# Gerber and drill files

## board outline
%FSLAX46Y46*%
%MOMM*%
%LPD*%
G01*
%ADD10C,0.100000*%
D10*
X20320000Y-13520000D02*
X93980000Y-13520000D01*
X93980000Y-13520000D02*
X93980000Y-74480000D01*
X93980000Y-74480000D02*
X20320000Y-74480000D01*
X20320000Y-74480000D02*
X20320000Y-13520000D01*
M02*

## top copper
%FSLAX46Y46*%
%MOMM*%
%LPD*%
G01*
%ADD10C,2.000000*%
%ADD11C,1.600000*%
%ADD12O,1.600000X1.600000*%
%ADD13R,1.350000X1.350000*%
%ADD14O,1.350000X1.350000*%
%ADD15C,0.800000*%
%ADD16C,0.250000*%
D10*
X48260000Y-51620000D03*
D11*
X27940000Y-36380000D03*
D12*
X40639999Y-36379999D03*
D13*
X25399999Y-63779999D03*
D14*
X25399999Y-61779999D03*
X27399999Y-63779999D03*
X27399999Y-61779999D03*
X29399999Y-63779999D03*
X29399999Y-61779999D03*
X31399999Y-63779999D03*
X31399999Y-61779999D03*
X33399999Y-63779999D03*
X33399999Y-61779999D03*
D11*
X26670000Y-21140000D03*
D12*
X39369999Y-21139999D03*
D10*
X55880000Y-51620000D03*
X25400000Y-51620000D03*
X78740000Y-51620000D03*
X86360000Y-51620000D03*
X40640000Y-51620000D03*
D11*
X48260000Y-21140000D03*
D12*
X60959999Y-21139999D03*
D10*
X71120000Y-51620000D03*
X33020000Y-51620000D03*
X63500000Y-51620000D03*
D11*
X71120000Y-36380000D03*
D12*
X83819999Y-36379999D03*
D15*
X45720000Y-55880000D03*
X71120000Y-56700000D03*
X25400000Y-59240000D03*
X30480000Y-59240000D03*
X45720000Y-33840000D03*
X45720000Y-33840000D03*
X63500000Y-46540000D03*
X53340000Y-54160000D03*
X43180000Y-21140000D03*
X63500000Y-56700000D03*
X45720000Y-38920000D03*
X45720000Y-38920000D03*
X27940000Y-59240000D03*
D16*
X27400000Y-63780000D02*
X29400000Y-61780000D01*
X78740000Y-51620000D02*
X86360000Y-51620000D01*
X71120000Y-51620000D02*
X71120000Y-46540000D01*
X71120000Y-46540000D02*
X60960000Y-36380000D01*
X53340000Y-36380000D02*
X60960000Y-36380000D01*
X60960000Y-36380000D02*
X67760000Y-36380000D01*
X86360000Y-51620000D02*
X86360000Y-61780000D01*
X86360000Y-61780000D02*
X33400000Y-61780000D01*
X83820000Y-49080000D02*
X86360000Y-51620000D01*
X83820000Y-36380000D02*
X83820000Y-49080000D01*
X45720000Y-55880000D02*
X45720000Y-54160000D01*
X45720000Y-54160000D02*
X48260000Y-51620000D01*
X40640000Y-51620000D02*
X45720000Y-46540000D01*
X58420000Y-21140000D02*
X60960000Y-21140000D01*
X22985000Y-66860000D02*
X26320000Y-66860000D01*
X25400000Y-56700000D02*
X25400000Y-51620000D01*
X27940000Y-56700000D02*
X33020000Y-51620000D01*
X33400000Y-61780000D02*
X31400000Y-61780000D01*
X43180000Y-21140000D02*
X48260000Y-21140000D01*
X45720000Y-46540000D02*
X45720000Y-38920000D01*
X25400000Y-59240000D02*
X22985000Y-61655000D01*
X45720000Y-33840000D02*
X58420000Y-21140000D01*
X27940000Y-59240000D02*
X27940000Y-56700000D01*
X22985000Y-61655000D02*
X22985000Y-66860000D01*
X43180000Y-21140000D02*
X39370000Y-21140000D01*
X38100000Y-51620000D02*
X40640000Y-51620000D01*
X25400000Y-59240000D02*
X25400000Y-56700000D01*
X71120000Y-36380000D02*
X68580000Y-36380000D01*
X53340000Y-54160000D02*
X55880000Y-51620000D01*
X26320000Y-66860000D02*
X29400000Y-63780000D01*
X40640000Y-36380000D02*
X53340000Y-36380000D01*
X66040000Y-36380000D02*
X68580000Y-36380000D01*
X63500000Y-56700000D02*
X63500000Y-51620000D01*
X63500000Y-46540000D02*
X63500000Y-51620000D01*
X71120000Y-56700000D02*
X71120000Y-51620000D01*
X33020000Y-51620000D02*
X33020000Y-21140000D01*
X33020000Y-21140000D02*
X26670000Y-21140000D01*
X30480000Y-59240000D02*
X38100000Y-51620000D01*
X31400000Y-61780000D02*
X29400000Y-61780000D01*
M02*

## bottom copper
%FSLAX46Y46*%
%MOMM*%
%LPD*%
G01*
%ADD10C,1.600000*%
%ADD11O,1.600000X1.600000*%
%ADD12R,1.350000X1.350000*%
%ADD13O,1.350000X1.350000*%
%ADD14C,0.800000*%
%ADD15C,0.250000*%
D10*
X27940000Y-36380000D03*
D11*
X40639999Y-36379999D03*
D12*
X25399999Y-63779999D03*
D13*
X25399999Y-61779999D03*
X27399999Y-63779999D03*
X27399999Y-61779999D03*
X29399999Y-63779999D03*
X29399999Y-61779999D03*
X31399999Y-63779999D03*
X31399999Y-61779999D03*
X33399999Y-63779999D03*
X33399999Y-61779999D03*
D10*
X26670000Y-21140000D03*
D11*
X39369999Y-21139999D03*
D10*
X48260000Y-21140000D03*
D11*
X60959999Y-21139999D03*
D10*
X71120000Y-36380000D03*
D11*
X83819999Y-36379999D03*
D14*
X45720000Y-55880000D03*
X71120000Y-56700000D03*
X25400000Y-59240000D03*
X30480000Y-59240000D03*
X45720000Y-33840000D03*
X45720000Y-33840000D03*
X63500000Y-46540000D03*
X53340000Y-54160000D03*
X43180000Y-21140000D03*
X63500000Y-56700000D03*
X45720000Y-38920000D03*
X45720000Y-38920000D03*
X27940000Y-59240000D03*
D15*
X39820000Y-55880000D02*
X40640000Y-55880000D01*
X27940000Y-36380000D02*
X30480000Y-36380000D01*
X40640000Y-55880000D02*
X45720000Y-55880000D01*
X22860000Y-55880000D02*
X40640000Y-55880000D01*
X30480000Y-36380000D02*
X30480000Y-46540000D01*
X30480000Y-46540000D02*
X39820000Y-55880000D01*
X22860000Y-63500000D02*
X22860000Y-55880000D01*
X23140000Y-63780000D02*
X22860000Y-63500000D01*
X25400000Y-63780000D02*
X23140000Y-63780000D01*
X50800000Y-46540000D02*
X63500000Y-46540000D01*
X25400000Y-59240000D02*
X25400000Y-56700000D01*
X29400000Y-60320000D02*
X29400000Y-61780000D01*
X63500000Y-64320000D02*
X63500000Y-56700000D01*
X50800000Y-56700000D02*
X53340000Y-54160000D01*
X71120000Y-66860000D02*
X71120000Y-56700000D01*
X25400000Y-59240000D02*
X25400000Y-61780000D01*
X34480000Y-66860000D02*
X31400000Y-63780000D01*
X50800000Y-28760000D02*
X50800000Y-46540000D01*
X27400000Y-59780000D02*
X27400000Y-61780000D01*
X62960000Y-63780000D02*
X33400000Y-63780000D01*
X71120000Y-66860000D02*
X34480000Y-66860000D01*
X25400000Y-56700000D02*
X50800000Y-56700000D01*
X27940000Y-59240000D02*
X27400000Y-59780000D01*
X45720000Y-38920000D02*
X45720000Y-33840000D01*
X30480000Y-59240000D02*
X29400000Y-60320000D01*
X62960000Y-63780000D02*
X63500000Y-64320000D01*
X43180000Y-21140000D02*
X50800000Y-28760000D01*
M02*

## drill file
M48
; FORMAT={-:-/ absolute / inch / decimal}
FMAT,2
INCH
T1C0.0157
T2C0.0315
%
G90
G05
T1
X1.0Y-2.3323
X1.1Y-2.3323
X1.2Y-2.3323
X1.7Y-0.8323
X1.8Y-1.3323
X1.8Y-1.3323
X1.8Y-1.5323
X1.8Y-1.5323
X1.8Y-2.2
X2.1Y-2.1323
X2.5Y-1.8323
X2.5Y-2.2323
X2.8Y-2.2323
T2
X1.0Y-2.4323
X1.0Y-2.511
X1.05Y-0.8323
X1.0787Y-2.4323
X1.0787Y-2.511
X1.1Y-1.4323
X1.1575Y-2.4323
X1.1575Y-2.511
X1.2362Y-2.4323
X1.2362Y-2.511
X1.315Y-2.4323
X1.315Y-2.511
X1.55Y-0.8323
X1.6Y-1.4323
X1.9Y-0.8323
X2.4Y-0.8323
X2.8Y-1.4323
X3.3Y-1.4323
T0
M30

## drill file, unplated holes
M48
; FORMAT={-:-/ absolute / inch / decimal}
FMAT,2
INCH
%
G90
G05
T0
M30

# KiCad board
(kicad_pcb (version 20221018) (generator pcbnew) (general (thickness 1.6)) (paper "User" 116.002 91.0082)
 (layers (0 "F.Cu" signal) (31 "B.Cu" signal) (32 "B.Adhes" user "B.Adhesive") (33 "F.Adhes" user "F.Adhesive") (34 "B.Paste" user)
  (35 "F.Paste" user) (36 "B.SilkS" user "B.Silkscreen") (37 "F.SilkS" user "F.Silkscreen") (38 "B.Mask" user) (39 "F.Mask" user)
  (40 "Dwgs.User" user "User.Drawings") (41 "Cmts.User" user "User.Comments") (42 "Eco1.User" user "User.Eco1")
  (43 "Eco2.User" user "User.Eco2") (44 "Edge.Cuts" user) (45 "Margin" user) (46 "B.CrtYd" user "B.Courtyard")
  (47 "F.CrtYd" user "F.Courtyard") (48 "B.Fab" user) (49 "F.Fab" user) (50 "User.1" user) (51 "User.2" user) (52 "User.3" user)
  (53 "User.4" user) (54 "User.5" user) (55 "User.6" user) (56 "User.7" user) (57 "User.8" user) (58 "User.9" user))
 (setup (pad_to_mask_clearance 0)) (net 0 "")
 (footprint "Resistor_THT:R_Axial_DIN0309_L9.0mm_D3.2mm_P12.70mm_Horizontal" (layer "F.Cu") (at 27.94 36.38)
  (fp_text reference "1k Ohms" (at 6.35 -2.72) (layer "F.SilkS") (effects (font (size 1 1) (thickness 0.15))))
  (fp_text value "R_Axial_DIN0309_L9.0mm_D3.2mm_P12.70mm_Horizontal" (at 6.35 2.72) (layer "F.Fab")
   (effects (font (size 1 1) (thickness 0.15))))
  (pad "1" thru_hole circle (at 0 0) (size 1.6 1.6) (drill 0.8) (layers "*.Cu" "*.Mask"))
  (pad "2" thru_hole oval (at 12.7 0) (size 1.6 1.6) (drill 0.8) (layers "*.Cu" "*.Mask")))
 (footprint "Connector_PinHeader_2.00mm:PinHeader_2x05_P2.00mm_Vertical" (layer "F.Cu") (at 25.4 63.78 90)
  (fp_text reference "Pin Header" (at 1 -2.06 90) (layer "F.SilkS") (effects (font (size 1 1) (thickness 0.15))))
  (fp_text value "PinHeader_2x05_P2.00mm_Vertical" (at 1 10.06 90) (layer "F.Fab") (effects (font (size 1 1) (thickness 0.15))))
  (pad "1" thru_hole rect (at 0 0 90) (size 1.35 1.35) (drill 0.8) (layers "*.Cu" "*.Mask"))
  (pad "2" thru_hole oval (at 2 0 90) (size 1.35 1.35) (drill 0.8) (layers "*.Cu" "*.Mask"))
  (pad "3" thru_hole oval (at 0 2 90) (size 1.35 1.35) (drill 0.8) (layers "*.Cu" "*.Mask"))
  (pad "4" thru_hole oval (at 2 2 90) (size 1.35 1.35) (drill 0.8) (layers "*.Cu" "*.Mask"))
  (pad "5" thru_hole oval (at 0 4 90) (size 1.35 1.35) (drill 0.8) (layers "*.Cu" "*.Mask"))
  (pad "6" thru_hole oval (at 2 4 90) (size 1.35 1.35) (drill 0.8) (layers "*.Cu" "*.Mask"))
  (pad "7" thru_hole oval (at 0 6 90) (size 1.35 1.35) (drill 0.8) (layers "*.Cu" "*.Mask"))
  (pad "8" thru_hole oval (at 2 6 90) (size 1.35 1.35) (drill 0.8) (layers "*.Cu" "*.Mask"))
  (pad "9" thru_hole oval (at 0 8 90) (size 1.35 1.35) (drill 0.8) (layers "*.Cu" "*.Mask"))
  (pad "10" thru_hole oval (at 2 8 90) (size 1.35 1.35) (drill 0.8) (layers "*.Cu" "*.Mask")))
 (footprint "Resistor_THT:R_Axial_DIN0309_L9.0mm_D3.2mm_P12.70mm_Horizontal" (layer "F.Cu") (at 26.67 21.14)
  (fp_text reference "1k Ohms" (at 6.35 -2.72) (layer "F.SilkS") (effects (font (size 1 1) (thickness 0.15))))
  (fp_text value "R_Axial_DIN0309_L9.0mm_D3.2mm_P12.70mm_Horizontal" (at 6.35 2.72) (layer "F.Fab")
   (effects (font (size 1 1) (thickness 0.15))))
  (pad "1" thru_hole circle (at 0 0) (size 1.6 1.6) (drill 0.8) (layers "*.Cu" "*.Mask"))
  (pad "2" thru_hole oval (at 12.7 0) (size 1.6 1.6) (drill 0.8) (layers "*.Cu" "*.Mask")))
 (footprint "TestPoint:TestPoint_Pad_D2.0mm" (layer "F.Cu") (at 55.88 51.62)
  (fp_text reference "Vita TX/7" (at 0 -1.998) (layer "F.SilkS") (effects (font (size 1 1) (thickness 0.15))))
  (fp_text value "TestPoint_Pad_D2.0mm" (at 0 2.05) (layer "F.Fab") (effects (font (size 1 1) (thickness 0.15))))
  (pad "1" smd circle (at 0 0) (size 2 2) (layers "F.Cu" "F.Mask")))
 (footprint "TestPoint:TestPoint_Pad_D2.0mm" (layer "F.Cu") (at 48.26 51.62)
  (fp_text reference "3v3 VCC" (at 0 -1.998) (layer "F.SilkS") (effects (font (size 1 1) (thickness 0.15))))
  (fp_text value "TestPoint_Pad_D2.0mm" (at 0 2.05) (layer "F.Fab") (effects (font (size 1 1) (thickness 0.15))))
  (pad "1" smd circle (at 0 0) (size 2 2) (layers "F.Cu" "F.Mask")))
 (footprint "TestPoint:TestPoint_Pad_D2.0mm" (layer "F.Cu") (at 25.4 51.62)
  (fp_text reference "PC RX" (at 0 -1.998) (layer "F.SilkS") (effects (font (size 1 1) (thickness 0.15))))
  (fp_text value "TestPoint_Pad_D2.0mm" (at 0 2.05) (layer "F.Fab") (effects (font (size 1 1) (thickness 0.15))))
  (pad "1" smd circle (at 0 0) (size 2 2) (layers "F.Cu" "F.Mask")))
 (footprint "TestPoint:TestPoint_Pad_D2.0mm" (layer "F.Cu") (at 78.74 51.62)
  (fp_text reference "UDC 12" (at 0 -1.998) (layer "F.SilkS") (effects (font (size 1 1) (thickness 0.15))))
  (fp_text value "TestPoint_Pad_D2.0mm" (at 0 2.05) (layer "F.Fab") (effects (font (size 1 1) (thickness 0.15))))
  (pad "1" smd circle (at 0 0) (size 2 2) (layers "F.Cu" "F.Mask")))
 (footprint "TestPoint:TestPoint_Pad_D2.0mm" (layer "F.Cu") (at 86.36 51.62)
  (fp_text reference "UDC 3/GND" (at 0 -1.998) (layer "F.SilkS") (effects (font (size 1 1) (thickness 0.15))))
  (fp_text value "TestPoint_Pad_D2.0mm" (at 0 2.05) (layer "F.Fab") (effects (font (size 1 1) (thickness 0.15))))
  (pad "1" smd circle (at 0 0) (size 2 2) (layers "F.Cu" "F.Mask")))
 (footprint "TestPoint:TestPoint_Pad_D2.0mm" (layer "F.Cu") (at 40.64 51.62)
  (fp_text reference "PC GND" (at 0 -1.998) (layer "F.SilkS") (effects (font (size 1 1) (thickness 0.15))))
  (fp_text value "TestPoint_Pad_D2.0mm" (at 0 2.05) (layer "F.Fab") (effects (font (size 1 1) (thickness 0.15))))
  (pad "1" smd circle (at 0 0) (size 2 2) (layers "F.Cu" "F.Mask")))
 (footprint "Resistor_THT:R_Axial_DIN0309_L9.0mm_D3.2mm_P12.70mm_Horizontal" (layer "F.Cu") (at 48.26 21.14)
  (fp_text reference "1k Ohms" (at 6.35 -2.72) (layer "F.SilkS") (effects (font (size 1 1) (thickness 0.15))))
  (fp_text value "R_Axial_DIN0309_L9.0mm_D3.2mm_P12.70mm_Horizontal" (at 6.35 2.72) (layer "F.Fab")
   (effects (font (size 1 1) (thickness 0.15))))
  (pad "1" thru_hole circle (at 0 0) (size 1.6 1.6) (drill 0.8) (layers "*.Cu" "*.Mask"))
  (pad "2" thru_hole oval (at 12.7 0) (size 1.6 1.6) (drill 0.8) (layers "*.Cu" "*.Mask")))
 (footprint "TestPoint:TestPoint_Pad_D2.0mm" (layer "F.Cu") (at 71.12 51.62)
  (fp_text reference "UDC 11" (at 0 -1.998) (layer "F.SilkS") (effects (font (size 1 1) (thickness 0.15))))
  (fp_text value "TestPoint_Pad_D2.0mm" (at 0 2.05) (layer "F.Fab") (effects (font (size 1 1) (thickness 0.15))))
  (pad "1" smd circle (at 0 0) (size 2 2) (layers "F.Cu" "F.Mask")))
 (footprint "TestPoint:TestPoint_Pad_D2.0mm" (layer "F.Cu") (at 33.02 51.62)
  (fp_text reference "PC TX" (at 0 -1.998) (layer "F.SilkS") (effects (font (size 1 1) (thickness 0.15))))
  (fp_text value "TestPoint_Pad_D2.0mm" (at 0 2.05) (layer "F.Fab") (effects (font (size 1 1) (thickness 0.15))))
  (pad "1" smd circle (at 0 0) (size 2 2) (layers "F.Cu" "F.Mask")))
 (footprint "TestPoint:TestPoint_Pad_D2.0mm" (layer "F.Cu") (at 63.5 51.62)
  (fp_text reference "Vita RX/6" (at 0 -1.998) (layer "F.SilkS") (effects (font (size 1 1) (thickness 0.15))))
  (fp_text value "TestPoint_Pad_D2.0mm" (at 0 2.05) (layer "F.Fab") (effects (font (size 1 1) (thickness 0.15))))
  (pad "1" smd circle (at 0 0) (size 2 2) (layers "F.Cu" "F.Mask")))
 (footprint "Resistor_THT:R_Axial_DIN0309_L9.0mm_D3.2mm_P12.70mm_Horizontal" (layer "F.Cu") (at 71.12 36.38)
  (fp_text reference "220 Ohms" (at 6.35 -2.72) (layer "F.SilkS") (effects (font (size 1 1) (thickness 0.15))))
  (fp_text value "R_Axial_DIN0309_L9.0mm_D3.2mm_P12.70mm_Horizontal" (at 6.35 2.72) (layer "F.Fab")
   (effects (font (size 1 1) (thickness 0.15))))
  (pad "1" thru_hole circle (at 0 0) (size 1.6 1.6) (drill 0.8) (layers "*.Cu" "*.Mask"))
  (pad "2" thru_hole oval (at 12.7 0) (size 1.6 1.6) (drill 0.8) (layers "*.Cu" "*.Mask")))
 (gr_rect (start 20.32 13.52) (end 93.98 74.48) (stroke (width 0.1) (type default)) (fill none) (layer "Edge.Cuts"))
 (segment (start 40.64 51.62) (end 45.72 46.54) (width 0.25) (layer "F.Cu") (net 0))
 (segment (start 58.42 21.14) (end 60.96 21.14) (width 0.25) (layer "F.Cu") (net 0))
 (segment (start 22.985 66.86) (end 26.32 66.86) (width 0.25) (layer "F.Cu") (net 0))
 (segment (start 25.4 56.7) (end 25.4 51.62) (width 0.25) (layer "F.Cu") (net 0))
 (segment (start 83.82 49.08) (end 86.36 51.62) (width 0.25) (layer "F.Cu") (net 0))
 (segment (start 27.94 56.7) (end 33.02 51.62) (width 0.25) (layer "F.Cu") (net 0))
 (segment (start 33.4 61.78) (end 31.4 61.78) (width 0.25) (layer "F.Cu") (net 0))
 (segment (start 43.18 21.14) (end 48.26 21.14) (width 0.25) (layer "F.Cu") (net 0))
 (segment (start 45.72 46.54) (end 45.72 38.92) (width 0.25) (layer "F.Cu") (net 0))
 (segment (start 45.72 55.88) (end 45.72 54.16) (width 0.25) (layer "F.Cu") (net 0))
 (segment (start 60.96 36.38) (end 67.76 36.38) (width 0.25) (layer "F.Cu") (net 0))
 (segment (start 25.4 59.24) (end 22.985 61.655) (width 0.25) (layer "F.Cu") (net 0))
 (segment (start 45.72 54.16) (end 48.26 51.62) (width 0.25) (layer "F.Cu") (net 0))
 (segment (start 45.72 33.84) (end 58.42 21.14) (width 0.25) (layer "F.Cu") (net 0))
 (segment (start 27.94 59.24) (end 27.94 56.7) (width 0.25) (layer "F.Cu") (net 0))
 (segment (start 22.985 61.655) (end 22.985 66.86) (width 0.25) (layer "F.Cu") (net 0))
 (segment (start 43.18 21.14) (end 39.37 21.14) (width 0.25) (layer "F.Cu") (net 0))
 (segment (start 38.1 51.62) (end 40.64 51.62) (width 0.25) (layer "F.Cu") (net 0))
 (segment (start 25.4 59.24) (end 25.4 56.7) (width 0.25) (layer "F.Cu") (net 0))
 (segment (start 78.74 51.62) (end 86.36 51.62) (width 0.25) (layer "F.Cu") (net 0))
 (segment (start 71.12 36.38) (end 68.58 36.38) (width 0.25) (layer "F.Cu") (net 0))
 (segment (start 53.34 54.16) (end 55.88 51.62) (width 0.25) (layer "F.Cu") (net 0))
 (segment (start 26.32 66.86) (end 29.4 63.78) (width 0.25) (layer "F.Cu") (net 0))
 (segment (start 40.64 36.38) (end 53.34 36.38) (width 0.25) (layer "F.Cu") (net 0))
 (segment (start 86.36 61.78) (end 33.4 61.78) (width 0.25) (layer "F.Cu") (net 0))
 (segment (start 27.4 63.78) (end 29.4 61.78) (width 0.25) (layer "F.Cu") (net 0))
 (segment (start 53.34 36.38) (end 60.96 36.38) (width 0.25) (layer "F.Cu") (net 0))
 (segment (start 66.04 36.38) (end 68.58 36.38) (width 0.25) (layer "F.Cu") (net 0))
 (segment (start 83.82 36.38) (end 83.82 49.08) (width 0.25) (layer "F.Cu") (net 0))
 (segment (start 63.5 56.7) (end 63.5 51.62) (width 0.25) (layer "F.Cu") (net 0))
 (segment (start 71.12 51.62) (end 71.12 46.54) (width 0.25) (layer "F.Cu") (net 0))
 (segment (start 63.5 46.54) (end 63.5 51.62) (width 0.25) (layer "F.Cu") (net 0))
 (segment (start 71.12 56.7) (end 71.12 51.62) (width 0.25) (layer "F.Cu") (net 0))
 (segment (start 71.12 46.54) (end 60.96 36.38) (width 0.25) (layer "F.Cu") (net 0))
 (segment (start 33.02 51.62) (end 33.02 21.14) (width 0.25) (layer "F.Cu") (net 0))
 (segment (start 33.02 21.14) (end 26.67 21.14) (width 0.25) (layer "F.Cu") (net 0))
 (segment (start 86.36 51.62) (end 86.36 61.78) (width 0.25) (layer "F.Cu") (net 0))
 (segment (start 30.48 59.24) (end 38.1 51.62) (width 0.25) (layer "F.Cu") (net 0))
 (segment (start 31.4 61.78) (end 29.4 61.78) (width 0.25) (layer "F.Cu") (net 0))
 (via (at 71.12 56.7) (size 0.8) (drill 0.4) (layers "F.Cu" "B.Cu") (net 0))
 (via (at 25.4 59.24) (size 0.8) (drill 0.4) (layers "F.Cu" "B.Cu") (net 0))
 (via (at 30.48 59.24) (size 0.8) (drill 0.4) (layers "F.Cu" "B.Cu") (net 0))
 (via (at 45.72 33.84) (size 0.8) (drill 0.4) (layers "F.Cu" "B.Cu") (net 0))
 (via (at 45.72 33.84) (size 0.8) (drill 0.4) (layers "F.Cu" "B.Cu") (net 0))
 (via (at 63.5 46.54) (size 0.8) (drill 0.4) (layers "F.Cu" "B.Cu") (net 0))
 (via (at 53.34 54.16) (size 0.8) (drill 0.4) (layers "F.Cu" "B.Cu") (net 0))
 (via (at 43.18 21.14) (size 0.8) (drill 0.4) (layers "F.Cu" "B.Cu") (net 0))
 (via (at 63.5 56.7) (size 0.8) (drill 0.4) (layers "F.Cu" "B.Cu") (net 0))
 (via (at 45.72 38.92) (size 0.8) (drill 0.4) (layers "F.Cu" "B.Cu") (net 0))
 (via (at 45.72 38.92) (size 0.8) (drill 0.4) (layers "F.Cu" "B.Cu") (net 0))
 (via (at 27.94 59.24) (size 0.8) (drill 0.4) (layers "F.Cu" "B.Cu") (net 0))
 (via (at 45.72 55.88) (size 0.8) (drill 0.4) (layers "F.Cu" "B.Cu") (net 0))
 (segment (start 27.94 36.38) (end 30.48 36.38) (width 0.25) (layer "B.Cu") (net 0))
 (segment (start 50.8 46.54) (end 63.5 46.54) (width 0.25) (layer "B.Cu") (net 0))
 (segment (start 40.64 55.88) (end 45.72 55.88) (width 0.25) (layer "B.Cu") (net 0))
 (segment (start 25.4 59.24) (end 25.4 56.7) (width 0.25) (layer "B.Cu") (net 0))
 (segment (start 30.48 46.54) (end 39.82 55.88) (width 0.25) (layer "B.Cu") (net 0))
 (segment (start 29.4 60.32) (end 29.4 61.78) (width 0.25) (layer "B.Cu") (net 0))
 (segment (start 63.5 64.32) (end 63.5 56.7) (width 0.25) (layer "B.Cu") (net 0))
 (segment (start 22.86 55.88) (end 40.64 55.88) (width 0.25) (layer "B.Cu") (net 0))
 (segment (start 25.4 63.78) (end 23.14 63.78) (width 0.25) (layer "B.Cu") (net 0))
 (segment (start 50.8 56.7) (end 53.34 54.16) (width 0.25) (layer "B.Cu") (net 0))
 (segment (start 71.12 66.86) (end 71.12 56.7) (width 0.25) (layer "B.Cu") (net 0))
 (segment (start 25.4 59.24) (end 25.4 61.78) (width 0.25) (layer "B.Cu") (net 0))
 (segment (start 23.14 63.78) (end 22.86 63.5) (width 0.25) (layer "B.Cu") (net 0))
 (segment (start 34.48 66.86) (end 31.4 63.78) (width 0.25) (layer "B.Cu") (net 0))
 (segment (start 50.8 28.76) (end 50.8 46.54) (width 0.25) (layer "B.Cu") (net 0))
 (segment (start 27.4 59.78) (end 27.4 61.78) (width 0.25) (layer "B.Cu") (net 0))
 (segment (start 22.86 63.5) (end 22.86 55.88) (width 0.25) (layer "B.Cu") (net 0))
 (segment (start 62.96 63.78) (end 33.4 63.78) (width 0.25) (layer "B.Cu") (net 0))
 (segment (start 71.12 66.86) (end 34.48 66.86) (width 0.25) (layer "B.Cu") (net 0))
 (segment (start 25.4 56.7) (end 50.8 56.7) (width 0.25) (layer "B.Cu") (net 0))
 (segment (start 30.48 36.38) (end 30.48 46.54) (width 0.25) (layer "B.Cu") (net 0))
 (segment (start 39.82 55.88) (end 40.64 55.88) (width 0.25) (layer "B.Cu") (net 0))
 (segment (start 27.94 59.24) (end 27.4 59.78) (width 0.25) (layer "B.Cu") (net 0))
 (segment (start 45.72 38.92) (end 45.72 33.84) (width 0.25) (layer "B.Cu") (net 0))
 (segment (start 30.48 59.24) (end 29.4 60.32) (width 0.25) (layer "B.Cu") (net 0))
 (segment (start 62.96 63.78) (end 63.5 64.32) (width 0.25) (layer "B.Cu") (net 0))
 (segment (start 43.18 21.14) (end 50.8 28.76) (width 0.25) (layer "B.Cu") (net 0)))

